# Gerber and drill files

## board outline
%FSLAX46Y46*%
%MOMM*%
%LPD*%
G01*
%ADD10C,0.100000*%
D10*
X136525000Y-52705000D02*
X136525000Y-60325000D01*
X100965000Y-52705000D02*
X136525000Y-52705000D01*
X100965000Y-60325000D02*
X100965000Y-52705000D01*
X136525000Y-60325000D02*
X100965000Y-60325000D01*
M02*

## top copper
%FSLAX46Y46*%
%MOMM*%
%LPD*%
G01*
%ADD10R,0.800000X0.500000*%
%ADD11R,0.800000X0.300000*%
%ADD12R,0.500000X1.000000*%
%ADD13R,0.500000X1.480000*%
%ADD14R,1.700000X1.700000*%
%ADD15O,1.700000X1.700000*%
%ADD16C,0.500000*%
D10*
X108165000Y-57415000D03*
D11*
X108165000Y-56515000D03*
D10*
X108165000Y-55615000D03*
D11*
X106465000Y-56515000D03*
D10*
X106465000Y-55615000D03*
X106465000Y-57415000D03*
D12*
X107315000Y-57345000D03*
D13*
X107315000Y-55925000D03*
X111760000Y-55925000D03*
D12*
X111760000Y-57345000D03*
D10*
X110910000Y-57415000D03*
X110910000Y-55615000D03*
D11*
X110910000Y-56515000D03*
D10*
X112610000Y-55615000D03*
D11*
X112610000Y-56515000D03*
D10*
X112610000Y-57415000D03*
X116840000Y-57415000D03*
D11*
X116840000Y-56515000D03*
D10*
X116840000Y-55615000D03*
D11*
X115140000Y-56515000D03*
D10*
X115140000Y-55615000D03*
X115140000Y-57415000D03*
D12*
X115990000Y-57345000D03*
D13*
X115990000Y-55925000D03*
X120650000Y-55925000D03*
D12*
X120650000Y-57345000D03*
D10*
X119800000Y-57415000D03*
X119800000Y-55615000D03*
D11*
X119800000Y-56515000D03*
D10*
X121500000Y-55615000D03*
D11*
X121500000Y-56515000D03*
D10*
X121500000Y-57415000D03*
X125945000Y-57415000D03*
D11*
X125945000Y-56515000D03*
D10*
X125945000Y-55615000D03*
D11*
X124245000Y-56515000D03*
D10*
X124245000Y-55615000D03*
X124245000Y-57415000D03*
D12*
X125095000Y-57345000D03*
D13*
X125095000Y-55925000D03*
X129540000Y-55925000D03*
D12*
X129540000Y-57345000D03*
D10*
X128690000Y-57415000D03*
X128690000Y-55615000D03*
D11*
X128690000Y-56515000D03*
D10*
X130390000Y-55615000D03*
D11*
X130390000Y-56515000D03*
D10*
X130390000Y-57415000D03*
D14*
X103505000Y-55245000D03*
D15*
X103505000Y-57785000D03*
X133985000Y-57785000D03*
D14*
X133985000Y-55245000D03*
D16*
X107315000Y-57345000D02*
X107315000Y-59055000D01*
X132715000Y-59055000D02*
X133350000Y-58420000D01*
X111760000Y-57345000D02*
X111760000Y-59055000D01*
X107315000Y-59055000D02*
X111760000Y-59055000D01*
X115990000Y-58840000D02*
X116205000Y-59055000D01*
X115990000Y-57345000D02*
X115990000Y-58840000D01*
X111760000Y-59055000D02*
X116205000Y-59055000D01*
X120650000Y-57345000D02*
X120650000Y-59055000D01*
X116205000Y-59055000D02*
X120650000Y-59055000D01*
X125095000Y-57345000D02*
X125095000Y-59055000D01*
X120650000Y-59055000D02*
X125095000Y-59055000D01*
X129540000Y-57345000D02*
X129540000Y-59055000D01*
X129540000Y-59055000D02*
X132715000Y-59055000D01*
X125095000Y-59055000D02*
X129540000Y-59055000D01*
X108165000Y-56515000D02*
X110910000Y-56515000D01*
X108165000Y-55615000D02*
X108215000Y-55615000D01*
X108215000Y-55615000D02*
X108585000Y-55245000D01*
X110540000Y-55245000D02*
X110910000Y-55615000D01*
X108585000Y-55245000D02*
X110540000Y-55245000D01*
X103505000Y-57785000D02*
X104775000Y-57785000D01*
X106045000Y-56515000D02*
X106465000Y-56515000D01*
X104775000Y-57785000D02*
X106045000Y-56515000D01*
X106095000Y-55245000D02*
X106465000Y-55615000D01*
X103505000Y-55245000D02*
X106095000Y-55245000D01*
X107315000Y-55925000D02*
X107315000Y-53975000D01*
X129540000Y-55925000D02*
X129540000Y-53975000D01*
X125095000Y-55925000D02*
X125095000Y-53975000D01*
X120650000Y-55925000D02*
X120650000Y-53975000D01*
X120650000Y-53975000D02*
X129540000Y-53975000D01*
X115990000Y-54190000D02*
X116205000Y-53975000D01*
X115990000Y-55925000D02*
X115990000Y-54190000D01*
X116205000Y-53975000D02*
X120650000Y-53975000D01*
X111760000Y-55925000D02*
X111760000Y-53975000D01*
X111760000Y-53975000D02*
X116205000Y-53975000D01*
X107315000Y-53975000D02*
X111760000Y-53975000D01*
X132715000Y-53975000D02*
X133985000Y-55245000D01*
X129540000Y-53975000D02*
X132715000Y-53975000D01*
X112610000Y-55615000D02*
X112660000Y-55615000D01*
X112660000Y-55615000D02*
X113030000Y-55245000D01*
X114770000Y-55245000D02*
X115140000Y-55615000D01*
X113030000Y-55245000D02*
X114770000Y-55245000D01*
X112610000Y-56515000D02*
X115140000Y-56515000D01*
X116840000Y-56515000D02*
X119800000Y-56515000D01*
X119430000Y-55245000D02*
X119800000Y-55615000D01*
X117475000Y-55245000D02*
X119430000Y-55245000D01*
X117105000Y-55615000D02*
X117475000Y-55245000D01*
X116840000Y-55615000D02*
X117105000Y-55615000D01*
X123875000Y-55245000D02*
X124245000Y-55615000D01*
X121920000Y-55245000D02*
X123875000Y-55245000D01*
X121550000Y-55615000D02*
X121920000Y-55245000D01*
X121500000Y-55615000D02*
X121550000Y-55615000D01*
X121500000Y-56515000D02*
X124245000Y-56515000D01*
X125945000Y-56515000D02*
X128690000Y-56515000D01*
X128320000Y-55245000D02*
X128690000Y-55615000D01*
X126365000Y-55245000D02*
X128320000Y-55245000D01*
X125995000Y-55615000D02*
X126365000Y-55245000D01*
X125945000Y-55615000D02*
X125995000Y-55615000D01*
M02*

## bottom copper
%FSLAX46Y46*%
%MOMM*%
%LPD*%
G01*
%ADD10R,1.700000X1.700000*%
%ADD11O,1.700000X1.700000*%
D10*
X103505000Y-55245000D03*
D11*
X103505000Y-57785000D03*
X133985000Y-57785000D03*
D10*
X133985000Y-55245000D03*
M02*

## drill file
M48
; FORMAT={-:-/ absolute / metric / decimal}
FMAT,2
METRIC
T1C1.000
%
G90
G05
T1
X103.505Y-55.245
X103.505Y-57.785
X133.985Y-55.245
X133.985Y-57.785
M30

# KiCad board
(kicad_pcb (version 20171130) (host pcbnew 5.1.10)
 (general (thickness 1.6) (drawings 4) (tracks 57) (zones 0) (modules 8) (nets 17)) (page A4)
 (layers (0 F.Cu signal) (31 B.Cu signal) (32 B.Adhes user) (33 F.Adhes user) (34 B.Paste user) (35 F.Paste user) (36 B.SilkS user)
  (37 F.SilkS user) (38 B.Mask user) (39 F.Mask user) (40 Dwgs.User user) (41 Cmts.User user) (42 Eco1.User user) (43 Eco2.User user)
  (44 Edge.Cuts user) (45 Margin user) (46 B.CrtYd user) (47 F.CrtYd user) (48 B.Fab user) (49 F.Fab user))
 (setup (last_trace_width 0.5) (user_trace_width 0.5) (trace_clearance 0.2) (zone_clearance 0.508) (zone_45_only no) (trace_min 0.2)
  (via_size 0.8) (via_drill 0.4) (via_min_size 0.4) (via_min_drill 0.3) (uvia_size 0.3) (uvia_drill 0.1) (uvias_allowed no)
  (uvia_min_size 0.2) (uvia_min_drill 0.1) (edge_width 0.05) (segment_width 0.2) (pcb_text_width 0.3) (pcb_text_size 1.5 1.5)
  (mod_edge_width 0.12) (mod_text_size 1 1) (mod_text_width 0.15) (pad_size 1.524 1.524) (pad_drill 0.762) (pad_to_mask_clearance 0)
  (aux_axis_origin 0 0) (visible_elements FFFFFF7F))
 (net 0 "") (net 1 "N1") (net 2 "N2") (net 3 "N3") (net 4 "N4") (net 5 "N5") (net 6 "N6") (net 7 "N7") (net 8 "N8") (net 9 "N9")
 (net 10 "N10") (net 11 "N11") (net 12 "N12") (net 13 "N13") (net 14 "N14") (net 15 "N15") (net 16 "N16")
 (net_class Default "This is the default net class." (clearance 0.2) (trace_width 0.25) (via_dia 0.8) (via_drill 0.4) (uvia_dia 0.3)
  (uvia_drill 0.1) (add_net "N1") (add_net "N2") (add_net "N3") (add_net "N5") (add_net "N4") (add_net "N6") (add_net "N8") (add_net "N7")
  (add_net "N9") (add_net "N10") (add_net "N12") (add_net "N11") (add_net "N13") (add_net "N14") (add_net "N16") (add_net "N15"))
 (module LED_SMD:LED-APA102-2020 (layer F.Cu) (at 107.315 56.515 180)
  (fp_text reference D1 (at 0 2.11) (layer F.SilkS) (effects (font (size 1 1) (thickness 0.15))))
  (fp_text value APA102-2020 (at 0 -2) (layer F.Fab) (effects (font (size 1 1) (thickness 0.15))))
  (pad 1 smd rect (at -0.85 -0.9 180) (size 0.8 0.5) (layers F.Cu F.Paste F.Mask) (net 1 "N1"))
  (pad 2 smd rect (at -0.85 0 180) (size 0.8 0.3) (layers F.Cu F.Paste F.Mask) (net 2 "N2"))
  (pad 3 smd rect (at -0.85 0.9 180) (size 0.8 0.5) (layers F.Cu F.Paste F.Mask) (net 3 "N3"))
  (pad 5 smd rect (at 0.85 0 180) (size 0.8 0.3) (layers F.Cu F.Paste F.Mask) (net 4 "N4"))
  (pad 4 smd rect (at 0.85 0.9 180) (size 0.8 0.5) (layers F.Cu F.Paste F.Mask) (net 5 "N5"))
  (pad 6 smd rect (at 0.85 -0.9 180) (size 0.8 0.5) (layers F.Cu F.Paste F.Mask) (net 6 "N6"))
  (pad 1 smd rect (at 0 -0.83 270) (size 1 0.5) (layers F.Cu F.Paste F.Mask) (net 1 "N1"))
  (pad 6 smd rect (at 0 0.59 270) (size 1.48 0.5) (layers F.Cu F.Paste F.Mask) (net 6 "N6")))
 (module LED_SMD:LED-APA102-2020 (layer F.Cu) (at 111.76 56.515 180)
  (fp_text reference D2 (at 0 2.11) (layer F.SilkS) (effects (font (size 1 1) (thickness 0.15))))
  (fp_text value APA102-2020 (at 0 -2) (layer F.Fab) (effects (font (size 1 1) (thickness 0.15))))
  (pad 6 smd rect (at 0 0.59 270) (size 1.48 0.5) (layers F.Cu F.Paste F.Mask) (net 6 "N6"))
  (pad 1 smd rect (at 0 -0.83 270) (size 1 0.5) (layers F.Cu F.Paste F.Mask) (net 1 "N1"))
  (pad 6 smd rect (at 0.85 -0.9 180) (size 0.8 0.5) (layers F.Cu F.Paste F.Mask) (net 6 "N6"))
  (pad 4 smd rect (at 0.85 0.9 180) (size 0.8 0.5) (layers F.Cu F.Paste F.Mask) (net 3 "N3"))
  (pad 5 smd rect (at 0.85 0 180) (size 0.8 0.3) (layers F.Cu F.Paste F.Mask) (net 2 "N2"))
  (pad 3 smd rect (at -0.85 0.9 180) (size 0.8 0.5) (layers F.Cu F.Paste F.Mask) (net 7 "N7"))
  (pad 2 smd rect (at -0.85 0 180) (size 0.8 0.3) (layers F.Cu F.Paste F.Mask) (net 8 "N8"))
  (pad 1 smd rect (at -0.85 -0.9 180) (size 0.8 0.5) (layers F.Cu F.Paste F.Mask) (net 1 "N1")))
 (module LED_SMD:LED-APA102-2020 (layer F.Cu) (at 115.99 56.515 180)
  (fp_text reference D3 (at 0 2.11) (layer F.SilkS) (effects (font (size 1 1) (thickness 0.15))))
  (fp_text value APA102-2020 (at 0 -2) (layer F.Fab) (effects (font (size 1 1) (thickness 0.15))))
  (pad 1 smd rect (at -0.85 -0.9 180) (size 0.8 0.5) (layers F.Cu F.Paste F.Mask) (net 1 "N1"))
  (pad 2 smd rect (at -0.85 0 180) (size 0.8 0.3) (layers F.Cu F.Paste F.Mask) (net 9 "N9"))
  (pad 3 smd rect (at -0.85 0.9 180) (size 0.8 0.5) (layers F.Cu F.Paste F.Mask) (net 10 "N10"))
  (pad 5 smd rect (at 0.85 0 180) (size 0.8 0.3) (layers F.Cu F.Paste F.Mask) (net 8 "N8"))
  (pad 4 smd rect (at 0.85 0.9 180) (size 0.8 0.5) (layers F.Cu F.Paste F.Mask) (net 7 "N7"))
  (pad 6 smd rect (at 0.85 -0.9 180) (size 0.8 0.5) (layers F.Cu F.Paste F.Mask) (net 6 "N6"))
  (pad 1 smd rect (at 0 -0.83 270) (size 1 0.5) (layers F.Cu F.Paste F.Mask) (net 1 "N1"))
  (pad 6 smd rect (at 0 0.59 270) (size 1.48 0.5) (layers F.Cu F.Paste F.Mask) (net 6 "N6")))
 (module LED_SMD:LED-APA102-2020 (layer F.Cu) (at 120.65 56.515 180)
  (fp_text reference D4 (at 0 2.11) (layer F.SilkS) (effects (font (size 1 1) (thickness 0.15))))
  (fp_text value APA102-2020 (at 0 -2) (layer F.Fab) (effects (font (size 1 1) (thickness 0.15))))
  (pad 6 smd rect (at 0 0.59 270) (size 1.48 0.5) (layers F.Cu F.Paste F.Mask) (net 6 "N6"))
  (pad 1 smd rect (at 0 -0.83 270) (size 1 0.5) (layers F.Cu F.Paste F.Mask) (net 1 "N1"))
  (pad 6 smd rect (at 0.85 -0.9 180) (size 0.8 0.5) (layers F.Cu F.Paste F.Mask) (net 6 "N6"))
  (pad 4 smd rect (at 0.85 0.9 180) (size 0.8 0.5) (layers F.Cu F.Paste F.Mask) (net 10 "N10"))
  (pad 5 smd rect (at 0.85 0 180) (size 0.8 0.3) (layers F.Cu F.Paste F.Mask) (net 9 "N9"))
  (pad 3 smd rect (at -0.85 0.9 180) (size 0.8 0.5) (layers F.Cu F.Paste F.Mask) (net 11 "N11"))
  (pad 2 smd rect (at -0.85 0 180) (size 0.8 0.3) (layers F.Cu F.Paste F.Mask) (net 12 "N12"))
  (pad 1 smd rect (at -0.85 -0.9 180) (size 0.8 0.5) (layers F.Cu F.Paste F.Mask) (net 1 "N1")))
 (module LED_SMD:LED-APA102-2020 (layer F.Cu) (at 125.095 56.515 180)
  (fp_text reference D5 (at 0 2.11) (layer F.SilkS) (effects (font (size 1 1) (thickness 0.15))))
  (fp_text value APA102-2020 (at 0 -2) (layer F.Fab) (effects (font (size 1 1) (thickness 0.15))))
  (pad 1 smd rect (at -0.85 -0.9 180) (size 0.8 0.5) (layers F.Cu F.Paste F.Mask) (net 1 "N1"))
  (pad 2 smd rect (at -0.85 0 180) (size 0.8 0.3) (layers F.Cu F.Paste F.Mask) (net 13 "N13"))
  (pad 3 smd rect (at -0.85 0.9 180) (size 0.8 0.5) (layers F.Cu F.Paste F.Mask) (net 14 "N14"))
  (pad 5 smd rect (at 0.85 0 180) (size 0.8 0.3) (layers F.Cu F.Paste F.Mask) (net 12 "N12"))
  (pad 4 smd rect (at 0.85 0.9 180) (size 0.8 0.5) (layers F.Cu F.Paste F.Mask) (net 11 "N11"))
  (pad 6 smd rect (at 0.85 -0.9 180) (size 0.8 0.5) (layers F.Cu F.Paste F.Mask) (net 6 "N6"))
  (pad 1 smd rect (at 0 -0.83 270) (size 1 0.5) (layers F.Cu F.Paste F.Mask) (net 1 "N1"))
  (pad 6 smd rect (at 0 0.59 270) (size 1.48 0.5) (layers F.Cu F.Paste F.Mask) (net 6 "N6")))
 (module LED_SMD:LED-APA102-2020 (layer F.Cu) (at 129.54 56.515 180)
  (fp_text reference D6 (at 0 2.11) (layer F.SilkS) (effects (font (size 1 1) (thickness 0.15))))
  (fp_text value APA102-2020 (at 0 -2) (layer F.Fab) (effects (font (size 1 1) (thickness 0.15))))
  (pad 6 smd rect (at 0 0.59 270) (size 1.48 0.5) (layers F.Cu F.Paste F.Mask) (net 6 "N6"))
  (pad 1 smd rect (at 0 -0.83 270) (size 1 0.5) (layers F.Cu F.Paste F.Mask) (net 1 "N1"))
  (pad 6 smd rect (at 0.85 -0.9 180) (size 0.8 0.5) (layers F.Cu F.Paste F.Mask) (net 6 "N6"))
  (pad 4 smd rect (at 0.85 0.9 180) (size 0.8 0.5) (layers F.Cu F.Paste F.Mask) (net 14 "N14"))
  (pad 5 smd rect (at 0.85 0 180) (size 0.8 0.3) (layers F.Cu F.Paste F.Mask) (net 13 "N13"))
  (pad 3 smd rect (at -0.85 0.9 180) (size 0.8 0.5) (layers F.Cu F.Paste F.Mask) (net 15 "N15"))
  (pad 2 smd rect (at -0.85 0 180) (size 0.8 0.3) (layers F.Cu F.Paste F.Mask) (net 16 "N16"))
  (pad 1 smd rect (at -0.85 -0.9 180) (size 0.8 0.5) (layers F.Cu F.Paste F.Mask) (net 1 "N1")))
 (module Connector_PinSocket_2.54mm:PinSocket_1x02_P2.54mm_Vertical (layer B.Cu) (at 103.505 55.245 180)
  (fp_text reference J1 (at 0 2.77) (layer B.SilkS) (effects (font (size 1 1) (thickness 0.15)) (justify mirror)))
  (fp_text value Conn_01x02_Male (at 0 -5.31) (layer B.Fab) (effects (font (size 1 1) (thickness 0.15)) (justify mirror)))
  (pad 1 thru_hole rect (at 0 0 180) (size 1.7 1.7) (drill 1) (layers *.Cu *.Mask) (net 5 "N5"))
  (pad 2 thru_hole oval (at 0 -2.54 180) (size 1.7 1.7) (drill 1) (layers *.Cu *.Mask) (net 4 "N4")))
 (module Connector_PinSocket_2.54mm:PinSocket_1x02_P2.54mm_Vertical (layer B.Cu) (at 133.985 55.245 180)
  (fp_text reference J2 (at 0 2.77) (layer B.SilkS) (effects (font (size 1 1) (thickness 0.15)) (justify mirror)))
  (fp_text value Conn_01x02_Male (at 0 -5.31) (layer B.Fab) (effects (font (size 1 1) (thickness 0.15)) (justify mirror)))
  (pad 2 thru_hole oval (at 0 -2.54 180) (size 1.7 1.7) (drill 1) (layers *.Cu *.Mask) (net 1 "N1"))
  (pad 1 thru_hole rect (at 0 0 180) (size 1.7 1.7) (drill 1) (layers *.Cu *.Mask) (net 6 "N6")))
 (gr_line (start 136.525 52.705) (end 136.525 60.325) (layer Edge.Cuts) (width 0.1))
 (gr_line (start 100.965 52.705) (end 136.525 52.705) (layer Edge.Cuts) (width 0.1))
 (gr_line (start 100.965 60.325) (end 100.965 52.705) (layer Edge.Cuts) (width 0.1))
 (gr_line (start 136.525 60.325) (end 100.965 60.325) (layer Edge.Cuts) (width 0.1))
 (segment (start 107.315 57.345) (end 107.315 59.055) (width 0.5) (layer F.Cu) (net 1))
 (segment (start 132.715 59.055) (end 133.35 58.42) (width 0.5) (layer F.Cu) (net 1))
 (segment (start 111.76 57.345) (end 111.76 59.055) (width 0.5) (layer F.Cu) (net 1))
 (segment (start 107.315 59.055) (end 111.76 59.055) (width 0.5) (layer F.Cu) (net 1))
 (segment (start 115.99 58.84) (end 116.205 59.055) (width 0.5) (layer F.Cu) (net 1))
 (segment (start 115.99 57.345) (end 115.99 58.84) (width 0.5) (layer F.Cu) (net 1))
 (segment (start 111.76 59.055) (end 116.205 59.055) (width 0.5) (layer F.Cu) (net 1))
 (segment (start 120.65 57.345) (end 120.65 59.055) (width 0.5) (layer F.Cu) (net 1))
 (segment (start 116.205 59.055) (end 120.65 59.055) (width 0.5) (layer F.Cu) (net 1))
 (segment (start 125.095 57.345) (end 125.095 59.055) (width 0.5) (layer F.Cu) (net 1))
 (segment (start 120.65 59.055) (end 125.095 59.055) (width 0.5) (layer F.Cu) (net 1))
 (segment (start 129.54 57.345) (end 129.54 59.055) (width 0.5) (layer F.Cu) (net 1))
 (segment (start 129.54 59.055) (end 132.715 59.055) (width 0.5) (layer F.Cu) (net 1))
 (segment (start 125.095 59.055) (end 129.54 59.055) (width 0.5) (layer F.Cu) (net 1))
 (segment (start 108.165 56.515) (end 110.91 56.515) (width 0.5) (layer F.Cu) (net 2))
 (segment (start 108.165 55.615) (end 108.215 55.615) (width 0.5) (layer F.Cu) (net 3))
 (segment (start 108.215 55.615) (end 108.585 55.245) (width 0.5) (layer F.Cu) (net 3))
 (segment (start 110.54 55.245) (end 110.91 55.615) (width 0.5) (layer F.Cu) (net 3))
 (segment (start 108.585 55.245) (end 110.54 55.245) (width 0.5) (layer F.Cu) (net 3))
 (segment (start 103.505 57.785) (end 104.775 57.785) (width 0.5) (layer F.Cu) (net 4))
 (segment (start 106.045 56.515) (end 106.465 56.515) (width 0.5) (layer F.Cu) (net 4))
 (segment (start 104.775 57.785) (end 106.045 56.515) (width 0.5) (layer F.Cu) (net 4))
 (segment (start 106.095 55.245) (end 106.465 55.615) (width 0.5) (layer F.Cu) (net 5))
 (segment (start 103.505 55.245) (end 106.095 55.245) (width 0.5) (layer F.Cu) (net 5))
 (segment (start 107.315 55.925) (end 107.315 53.975) (width 0.5) (layer F.Cu) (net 6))
 (segment (start 129.54 55.925) (end 129.54 53.975) (width 0.5) (layer F.Cu) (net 6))
 (segment (start 125.095 55.925) (end 125.095 53.975) (width 0.5) (layer F.Cu) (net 6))
 (segment (start 120.65 55.925) (end 120.65 53.975) (width 0.5) (layer F.Cu) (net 6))
 (segment (start 120.65 53.975) (end 129.54 53.975) (width 0.5) (layer F.Cu) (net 6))
 (segment (start 115.99 54.19) (end 116.205 53.975) (width 0.5) (layer F.Cu) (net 6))
 (segment (start 115.99 55.925) (end 115.99 54.19) (width 0.5) (layer F.Cu) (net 6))
 (segment (start 116.205 53.975) (end 120.65 53.975) (width 0.5) (layer F.Cu) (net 6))
 (segment (start 111.76 55.925) (end 111.76 53.975) (width 0.5) (layer F.Cu) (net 6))
 (segment (start 111.76 53.975) (end 116.205 53.975) (width 0.5) (layer F.Cu) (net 6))
 (segment (start 107.315 53.975) (end 111.76 53.975) (width 0.5) (layer F.Cu) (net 6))
 (segment (start 132.715 53.975) (end 133.985 55.245) (width 0.5) (layer F.Cu) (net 6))
 (segment (start 129.54 53.975) (end 132.715 53.975) (width 0.5) (layer F.Cu) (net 6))
 (segment (start 112.61 55.615) (end 112.66 55.615) (width 0.5) (layer F.Cu) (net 7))
 (segment (start 112.66 55.615) (end 113.03 55.245) (width 0.5) (layer F.Cu) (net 7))
 (segment (start 114.77 55.245) (end 115.14 55.615) (width 0.5) (layer F.Cu) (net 7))
 (segment (start 113.03 55.245) (end 114.77 55.245) (width 0.5) (layer F.Cu) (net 7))
 (segment (start 112.61 56.515) (end 115.14 56.515) (width 0.5) (layer F.Cu) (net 8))
 (segment (start 116.84 56.515) (end 119.8 56.515) (width 0.5) (layer F.Cu) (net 9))
 (segment (start 119.43 55.245) (end 119.8 55.615) (width 0.5) (layer F.Cu) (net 10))
 (segment (start 117.475 55.245) (end 119.43 55.245) (width 0.5) (layer F.Cu) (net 10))
 (segment (start 117.105 55.615) (end 117.475 55.245) (width 0.5) (layer F.Cu) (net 10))
 (segment (start 116.84 55.615) (end 117.105 55.615) (width 0.5) (layer F.Cu) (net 10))
 (segment (start 123.875 55.245) (end 124.245 55.615) (width 0.5) (layer F.Cu) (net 11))
 (segment (start 121.92 55.245) (end 123.875 55.245) (width 0.5) (layer F.Cu) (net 11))
 (segment (start 121.55 55.615) (end 121.92 55.245) (width 0.5) (layer F.Cu) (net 11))
 (segment (start 121.5 55.615) (end 121.55 55.615) (width 0.5) (layer F.Cu) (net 11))
 (segment (start 121.5 56.515) (end 124.245 56.515) (width 0.5) (layer F.Cu) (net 12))
 (segment (start 125.945 56.515) (end 128.69 56.515) (width 0.5) (layer F.Cu) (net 13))
 (segment (start 128.32 55.245) (end 128.69 55.615) (width 0.5) (layer F.Cu) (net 14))
 (segment (start 126.365 55.245) (end 128.32 55.245) (width 0.5) (layer F.Cu) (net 14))
 (segment (start 125.995 55.615) (end 126.365 55.245) (width 0.5) (layer F.Cu) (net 14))
 (segment (start 125.945 55.615) (end 125.995 55.615) (width 0.5) (layer F.Cu) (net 14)))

